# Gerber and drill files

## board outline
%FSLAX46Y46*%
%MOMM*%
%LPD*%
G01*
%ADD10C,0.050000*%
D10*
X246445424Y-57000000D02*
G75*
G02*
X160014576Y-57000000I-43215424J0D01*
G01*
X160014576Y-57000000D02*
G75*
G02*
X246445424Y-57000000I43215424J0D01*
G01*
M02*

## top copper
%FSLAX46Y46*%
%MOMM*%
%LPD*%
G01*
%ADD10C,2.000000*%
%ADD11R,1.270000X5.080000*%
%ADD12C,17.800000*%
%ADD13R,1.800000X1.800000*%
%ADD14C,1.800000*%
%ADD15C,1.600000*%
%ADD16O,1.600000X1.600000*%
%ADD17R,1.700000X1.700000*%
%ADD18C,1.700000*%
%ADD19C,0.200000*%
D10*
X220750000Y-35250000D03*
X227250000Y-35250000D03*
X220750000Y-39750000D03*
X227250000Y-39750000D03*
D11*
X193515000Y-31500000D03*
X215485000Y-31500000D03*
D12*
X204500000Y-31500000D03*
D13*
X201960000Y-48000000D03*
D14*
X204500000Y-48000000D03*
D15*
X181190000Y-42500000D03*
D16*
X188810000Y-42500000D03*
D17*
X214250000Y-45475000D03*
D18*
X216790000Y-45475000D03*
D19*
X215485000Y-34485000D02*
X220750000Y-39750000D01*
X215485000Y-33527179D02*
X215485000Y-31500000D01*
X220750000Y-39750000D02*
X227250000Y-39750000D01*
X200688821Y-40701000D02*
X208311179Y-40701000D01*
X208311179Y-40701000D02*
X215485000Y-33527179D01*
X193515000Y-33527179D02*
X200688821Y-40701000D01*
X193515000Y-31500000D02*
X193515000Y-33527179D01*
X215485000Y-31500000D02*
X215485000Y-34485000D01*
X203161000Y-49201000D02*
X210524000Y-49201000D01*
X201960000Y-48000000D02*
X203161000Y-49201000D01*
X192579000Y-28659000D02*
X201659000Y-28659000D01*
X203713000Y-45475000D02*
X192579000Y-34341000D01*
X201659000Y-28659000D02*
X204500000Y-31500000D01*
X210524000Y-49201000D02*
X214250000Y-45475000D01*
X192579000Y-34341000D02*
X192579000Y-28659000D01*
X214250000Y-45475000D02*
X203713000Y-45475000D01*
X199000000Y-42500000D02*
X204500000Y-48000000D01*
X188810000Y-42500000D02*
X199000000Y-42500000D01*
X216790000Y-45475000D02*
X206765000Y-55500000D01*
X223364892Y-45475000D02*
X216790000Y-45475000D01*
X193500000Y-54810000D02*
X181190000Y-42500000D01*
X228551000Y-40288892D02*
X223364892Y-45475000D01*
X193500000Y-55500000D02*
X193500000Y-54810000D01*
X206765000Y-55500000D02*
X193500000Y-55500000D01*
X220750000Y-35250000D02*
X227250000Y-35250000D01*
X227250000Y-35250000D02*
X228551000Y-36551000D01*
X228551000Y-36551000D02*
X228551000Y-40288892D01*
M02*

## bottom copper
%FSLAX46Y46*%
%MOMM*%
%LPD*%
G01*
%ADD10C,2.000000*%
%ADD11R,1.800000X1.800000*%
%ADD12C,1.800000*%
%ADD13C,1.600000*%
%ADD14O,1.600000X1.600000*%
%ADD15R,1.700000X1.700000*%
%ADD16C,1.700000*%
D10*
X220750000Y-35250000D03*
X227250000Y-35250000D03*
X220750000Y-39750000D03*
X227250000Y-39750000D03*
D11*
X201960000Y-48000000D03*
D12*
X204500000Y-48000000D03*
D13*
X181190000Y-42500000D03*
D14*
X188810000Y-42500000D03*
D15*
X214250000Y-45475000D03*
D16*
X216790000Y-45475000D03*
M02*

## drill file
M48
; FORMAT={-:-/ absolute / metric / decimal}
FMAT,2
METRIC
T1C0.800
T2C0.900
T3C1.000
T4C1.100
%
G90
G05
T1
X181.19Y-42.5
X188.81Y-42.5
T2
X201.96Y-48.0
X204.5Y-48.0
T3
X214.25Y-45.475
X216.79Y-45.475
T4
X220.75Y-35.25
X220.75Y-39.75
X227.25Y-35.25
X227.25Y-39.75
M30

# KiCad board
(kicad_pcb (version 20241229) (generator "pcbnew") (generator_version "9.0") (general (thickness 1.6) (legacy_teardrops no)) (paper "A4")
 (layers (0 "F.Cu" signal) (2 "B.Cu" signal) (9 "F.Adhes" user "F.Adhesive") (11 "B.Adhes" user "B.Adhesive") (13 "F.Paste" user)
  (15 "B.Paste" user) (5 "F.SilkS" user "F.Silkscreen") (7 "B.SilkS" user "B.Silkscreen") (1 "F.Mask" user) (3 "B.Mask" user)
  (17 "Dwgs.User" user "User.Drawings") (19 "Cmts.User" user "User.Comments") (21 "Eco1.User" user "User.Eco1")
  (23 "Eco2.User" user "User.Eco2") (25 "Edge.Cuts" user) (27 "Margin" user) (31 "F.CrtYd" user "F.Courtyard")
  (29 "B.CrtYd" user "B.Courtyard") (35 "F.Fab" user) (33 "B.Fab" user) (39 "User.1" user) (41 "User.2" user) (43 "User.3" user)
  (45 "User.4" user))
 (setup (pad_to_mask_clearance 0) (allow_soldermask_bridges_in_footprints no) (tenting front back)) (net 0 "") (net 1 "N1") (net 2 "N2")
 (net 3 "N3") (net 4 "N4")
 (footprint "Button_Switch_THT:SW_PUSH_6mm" (layer "F.Cu") (at 220.75 35.25)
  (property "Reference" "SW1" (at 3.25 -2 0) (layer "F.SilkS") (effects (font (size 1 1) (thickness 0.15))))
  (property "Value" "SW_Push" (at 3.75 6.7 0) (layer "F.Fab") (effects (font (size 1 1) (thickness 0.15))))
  (pad "1" thru_hole circle (at 0 0 90) (size 2 2) (drill 1.1) (layers "*.Cu" "*.Mask") (remove_unused_layers no) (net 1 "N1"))
  (pad "1" thru_hole circle (at 6.5 0 90) (size 2 2) (drill 1.1) (layers "*.Cu" "*.Mask") (remove_unused_layers no) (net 1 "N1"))
  (pad "2" thru_hole circle (at 0 4.5 90) (size 2 2) (drill 1.1) (layers "*.Cu" "*.Mask") (remove_unused_layers no) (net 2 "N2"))
  (pad "2" thru_hole circle (at 6.5 4.5 90) (size 2 2) (drill 1.1) (layers "*.Cu" "*.Mask") (remove_unused_layers no) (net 2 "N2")))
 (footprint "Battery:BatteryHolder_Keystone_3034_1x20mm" (layer "F.Cu") (at 204.5 31.5)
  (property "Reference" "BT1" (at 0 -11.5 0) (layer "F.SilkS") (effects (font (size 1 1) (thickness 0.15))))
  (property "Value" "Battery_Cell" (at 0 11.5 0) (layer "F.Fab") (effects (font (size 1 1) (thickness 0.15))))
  (pad "1" smd rect (at -10.985 0) (size 1.27 5.08) (layers "F.Cu" "F.Mask" "F.Paste") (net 2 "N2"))
  (pad "1" smd rect (at 10.985 0) (size 1.27 5.08) (layers "F.Cu" "F.Mask" "F.Paste") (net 2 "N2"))
  (pad "2" smd circle (at 0 0) (size 17.8 17.8) (layers "F.Cu" "F.Mask") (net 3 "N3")))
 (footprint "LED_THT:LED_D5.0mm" (layer "F.Cu") (at 201.96 48)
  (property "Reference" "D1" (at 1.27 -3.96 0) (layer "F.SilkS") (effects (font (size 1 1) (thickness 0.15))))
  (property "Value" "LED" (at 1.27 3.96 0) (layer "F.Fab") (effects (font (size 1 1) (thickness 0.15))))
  (pad "1" thru_hole rect (at 0 0) (size 1.8 1.8) (drill 0.9) (layers "*.Cu" "*.Mask") (remove_unused_layers no) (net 3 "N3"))
  (pad "2" thru_hole circle (at 2.54 0) (size 1.8 1.8) (drill 0.9) (layers "*.Cu" "*.Mask") (remove_unused_layers no) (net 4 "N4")))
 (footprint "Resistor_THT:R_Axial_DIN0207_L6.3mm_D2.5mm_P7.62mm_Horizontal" (layer "F.Cu") (at 181.19 42.5)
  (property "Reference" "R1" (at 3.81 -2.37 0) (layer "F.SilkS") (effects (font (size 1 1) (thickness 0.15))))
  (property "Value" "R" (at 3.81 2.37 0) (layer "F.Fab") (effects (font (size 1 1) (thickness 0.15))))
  (pad "1" thru_hole circle (at 0 0) (size 1.6 1.6) (drill 0.8) (layers "*.Cu" "*.Mask") (remove_unused_layers no) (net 1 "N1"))
  (pad "2" thru_hole oval (at 7.62 0) (size 1.6 1.6) (drill 0.8) (layers "*.Cu" "*.Mask") (remove_unused_layers no) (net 4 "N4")))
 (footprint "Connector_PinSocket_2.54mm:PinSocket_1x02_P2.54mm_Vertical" (layer "F.Cu") (at 214.25 45.475 90)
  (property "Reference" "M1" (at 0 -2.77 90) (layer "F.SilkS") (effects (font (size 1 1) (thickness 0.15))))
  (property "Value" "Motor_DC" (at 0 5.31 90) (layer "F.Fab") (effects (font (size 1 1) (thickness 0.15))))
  (pad "1" thru_hole rect (at 0 0 90) (size 1.7 1.7) (drill 1) (layers "*.Cu" "*.Mask") (remove_unused_layers no) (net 3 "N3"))
  (pad "2" thru_hole circle (at 0 2.54 90) (size 1.7 1.7) (drill 1) (layers "*.Cu" "*.Mask") (remove_unused_layers no) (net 1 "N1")))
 (gr_circle (center 203.23 57) (end 241 78) (stroke (width 0.05) (type default)) (fill no) (layer "Edge.Cuts"))
 (segment (start 215.485 34.485) (end 220.75 39.75) (width 0.2) (layer "F.Cu") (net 2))
 (segment (start 215.485 33.527179) (end 215.485 31.5) (width 0.2) (layer "F.Cu") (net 2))
 (segment (start 220.75 39.75) (end 227.25 39.75) (width 0.2) (layer "F.Cu") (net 2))
 (segment (start 200.688821 40.701) (end 208.311179 40.701) (width 0.2) (layer "F.Cu") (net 2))
 (segment (start 208.311179 40.701) (end 215.485 33.527179) (width 0.2) (layer "F.Cu") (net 2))
 (segment (start 193.515 33.527179) (end 200.688821 40.701) (width 0.2) (layer "F.Cu") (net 2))
 (segment (start 193.515 31.5) (end 193.515 33.527179) (width 0.2) (layer "F.Cu") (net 2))
 (segment (start 215.485 31.5) (end 215.485 34.485) (width 0.2) (layer "F.Cu") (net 2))
 (segment (start 203.161 49.201) (end 210.524 49.201) (width 0.2) (layer "F.Cu") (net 3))
 (segment (start 201.96 48) (end 203.161 49.201) (width 0.2) (layer "F.Cu") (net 3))
 (segment (start 192.579 28.659) (end 201.659 28.659) (width 0.2) (layer "F.Cu") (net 3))
 (segment (start 203.713 45.475) (end 192.579 34.341) (width 0.2) (layer "F.Cu") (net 3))
 (segment (start 201.659 28.659) (end 204.5 31.5) (width 0.2) (layer "F.Cu") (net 3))
 (segment (start 210.524 49.201) (end 214.25 45.475) (width 0.2) (layer "F.Cu") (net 3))
 (segment (start 192.579 34.341) (end 192.579 28.659) (width 0.2) (layer "F.Cu") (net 3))
 (segment (start 214.25 45.475) (end 203.713 45.475) (width 0.2) (layer "F.Cu") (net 3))
 (segment (start 199 42.5) (end 204.5 48) (width 0.2) (layer "F.Cu") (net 4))
 (segment (start 188.81 42.5) (end 199 42.5) (width 0.2) (layer "F.Cu") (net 4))
 (segment (start 216.79 45.475) (end 206.765 55.5) (width 0.2) (layer "F.Cu") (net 1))
 (segment (start 223.364892 45.475) (end 216.79 45.475) (width 0.2) (layer "F.Cu") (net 1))
 (segment (start 193.5 54.81) (end 181.19 42.5) (width 0.2) (layer "F.Cu") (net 1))
 (segment (start 228.551 40.288892) (end 223.364892 45.475) (width 0.2) (layer "F.Cu") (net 1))
 (segment (start 193.5 55.5) (end 193.5 54.81) (width 0.2) (layer "F.Cu") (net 1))
 (segment (start 206.765 55.5) (end 193.5 55.5) (width 0.2) (layer "F.Cu") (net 1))
 (segment (start 220.75 35.25) (end 227.25 35.25) (width 0.2) (layer "F.Cu") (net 1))
 (segment (start 227.25 35.25) (end 228.551 36.551) (width 0.2) (layer "F.Cu") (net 1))
 (segment (start 228.551 36.551) (end 228.551 40.288892) (width 0.2) (layer "F.Cu") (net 1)))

